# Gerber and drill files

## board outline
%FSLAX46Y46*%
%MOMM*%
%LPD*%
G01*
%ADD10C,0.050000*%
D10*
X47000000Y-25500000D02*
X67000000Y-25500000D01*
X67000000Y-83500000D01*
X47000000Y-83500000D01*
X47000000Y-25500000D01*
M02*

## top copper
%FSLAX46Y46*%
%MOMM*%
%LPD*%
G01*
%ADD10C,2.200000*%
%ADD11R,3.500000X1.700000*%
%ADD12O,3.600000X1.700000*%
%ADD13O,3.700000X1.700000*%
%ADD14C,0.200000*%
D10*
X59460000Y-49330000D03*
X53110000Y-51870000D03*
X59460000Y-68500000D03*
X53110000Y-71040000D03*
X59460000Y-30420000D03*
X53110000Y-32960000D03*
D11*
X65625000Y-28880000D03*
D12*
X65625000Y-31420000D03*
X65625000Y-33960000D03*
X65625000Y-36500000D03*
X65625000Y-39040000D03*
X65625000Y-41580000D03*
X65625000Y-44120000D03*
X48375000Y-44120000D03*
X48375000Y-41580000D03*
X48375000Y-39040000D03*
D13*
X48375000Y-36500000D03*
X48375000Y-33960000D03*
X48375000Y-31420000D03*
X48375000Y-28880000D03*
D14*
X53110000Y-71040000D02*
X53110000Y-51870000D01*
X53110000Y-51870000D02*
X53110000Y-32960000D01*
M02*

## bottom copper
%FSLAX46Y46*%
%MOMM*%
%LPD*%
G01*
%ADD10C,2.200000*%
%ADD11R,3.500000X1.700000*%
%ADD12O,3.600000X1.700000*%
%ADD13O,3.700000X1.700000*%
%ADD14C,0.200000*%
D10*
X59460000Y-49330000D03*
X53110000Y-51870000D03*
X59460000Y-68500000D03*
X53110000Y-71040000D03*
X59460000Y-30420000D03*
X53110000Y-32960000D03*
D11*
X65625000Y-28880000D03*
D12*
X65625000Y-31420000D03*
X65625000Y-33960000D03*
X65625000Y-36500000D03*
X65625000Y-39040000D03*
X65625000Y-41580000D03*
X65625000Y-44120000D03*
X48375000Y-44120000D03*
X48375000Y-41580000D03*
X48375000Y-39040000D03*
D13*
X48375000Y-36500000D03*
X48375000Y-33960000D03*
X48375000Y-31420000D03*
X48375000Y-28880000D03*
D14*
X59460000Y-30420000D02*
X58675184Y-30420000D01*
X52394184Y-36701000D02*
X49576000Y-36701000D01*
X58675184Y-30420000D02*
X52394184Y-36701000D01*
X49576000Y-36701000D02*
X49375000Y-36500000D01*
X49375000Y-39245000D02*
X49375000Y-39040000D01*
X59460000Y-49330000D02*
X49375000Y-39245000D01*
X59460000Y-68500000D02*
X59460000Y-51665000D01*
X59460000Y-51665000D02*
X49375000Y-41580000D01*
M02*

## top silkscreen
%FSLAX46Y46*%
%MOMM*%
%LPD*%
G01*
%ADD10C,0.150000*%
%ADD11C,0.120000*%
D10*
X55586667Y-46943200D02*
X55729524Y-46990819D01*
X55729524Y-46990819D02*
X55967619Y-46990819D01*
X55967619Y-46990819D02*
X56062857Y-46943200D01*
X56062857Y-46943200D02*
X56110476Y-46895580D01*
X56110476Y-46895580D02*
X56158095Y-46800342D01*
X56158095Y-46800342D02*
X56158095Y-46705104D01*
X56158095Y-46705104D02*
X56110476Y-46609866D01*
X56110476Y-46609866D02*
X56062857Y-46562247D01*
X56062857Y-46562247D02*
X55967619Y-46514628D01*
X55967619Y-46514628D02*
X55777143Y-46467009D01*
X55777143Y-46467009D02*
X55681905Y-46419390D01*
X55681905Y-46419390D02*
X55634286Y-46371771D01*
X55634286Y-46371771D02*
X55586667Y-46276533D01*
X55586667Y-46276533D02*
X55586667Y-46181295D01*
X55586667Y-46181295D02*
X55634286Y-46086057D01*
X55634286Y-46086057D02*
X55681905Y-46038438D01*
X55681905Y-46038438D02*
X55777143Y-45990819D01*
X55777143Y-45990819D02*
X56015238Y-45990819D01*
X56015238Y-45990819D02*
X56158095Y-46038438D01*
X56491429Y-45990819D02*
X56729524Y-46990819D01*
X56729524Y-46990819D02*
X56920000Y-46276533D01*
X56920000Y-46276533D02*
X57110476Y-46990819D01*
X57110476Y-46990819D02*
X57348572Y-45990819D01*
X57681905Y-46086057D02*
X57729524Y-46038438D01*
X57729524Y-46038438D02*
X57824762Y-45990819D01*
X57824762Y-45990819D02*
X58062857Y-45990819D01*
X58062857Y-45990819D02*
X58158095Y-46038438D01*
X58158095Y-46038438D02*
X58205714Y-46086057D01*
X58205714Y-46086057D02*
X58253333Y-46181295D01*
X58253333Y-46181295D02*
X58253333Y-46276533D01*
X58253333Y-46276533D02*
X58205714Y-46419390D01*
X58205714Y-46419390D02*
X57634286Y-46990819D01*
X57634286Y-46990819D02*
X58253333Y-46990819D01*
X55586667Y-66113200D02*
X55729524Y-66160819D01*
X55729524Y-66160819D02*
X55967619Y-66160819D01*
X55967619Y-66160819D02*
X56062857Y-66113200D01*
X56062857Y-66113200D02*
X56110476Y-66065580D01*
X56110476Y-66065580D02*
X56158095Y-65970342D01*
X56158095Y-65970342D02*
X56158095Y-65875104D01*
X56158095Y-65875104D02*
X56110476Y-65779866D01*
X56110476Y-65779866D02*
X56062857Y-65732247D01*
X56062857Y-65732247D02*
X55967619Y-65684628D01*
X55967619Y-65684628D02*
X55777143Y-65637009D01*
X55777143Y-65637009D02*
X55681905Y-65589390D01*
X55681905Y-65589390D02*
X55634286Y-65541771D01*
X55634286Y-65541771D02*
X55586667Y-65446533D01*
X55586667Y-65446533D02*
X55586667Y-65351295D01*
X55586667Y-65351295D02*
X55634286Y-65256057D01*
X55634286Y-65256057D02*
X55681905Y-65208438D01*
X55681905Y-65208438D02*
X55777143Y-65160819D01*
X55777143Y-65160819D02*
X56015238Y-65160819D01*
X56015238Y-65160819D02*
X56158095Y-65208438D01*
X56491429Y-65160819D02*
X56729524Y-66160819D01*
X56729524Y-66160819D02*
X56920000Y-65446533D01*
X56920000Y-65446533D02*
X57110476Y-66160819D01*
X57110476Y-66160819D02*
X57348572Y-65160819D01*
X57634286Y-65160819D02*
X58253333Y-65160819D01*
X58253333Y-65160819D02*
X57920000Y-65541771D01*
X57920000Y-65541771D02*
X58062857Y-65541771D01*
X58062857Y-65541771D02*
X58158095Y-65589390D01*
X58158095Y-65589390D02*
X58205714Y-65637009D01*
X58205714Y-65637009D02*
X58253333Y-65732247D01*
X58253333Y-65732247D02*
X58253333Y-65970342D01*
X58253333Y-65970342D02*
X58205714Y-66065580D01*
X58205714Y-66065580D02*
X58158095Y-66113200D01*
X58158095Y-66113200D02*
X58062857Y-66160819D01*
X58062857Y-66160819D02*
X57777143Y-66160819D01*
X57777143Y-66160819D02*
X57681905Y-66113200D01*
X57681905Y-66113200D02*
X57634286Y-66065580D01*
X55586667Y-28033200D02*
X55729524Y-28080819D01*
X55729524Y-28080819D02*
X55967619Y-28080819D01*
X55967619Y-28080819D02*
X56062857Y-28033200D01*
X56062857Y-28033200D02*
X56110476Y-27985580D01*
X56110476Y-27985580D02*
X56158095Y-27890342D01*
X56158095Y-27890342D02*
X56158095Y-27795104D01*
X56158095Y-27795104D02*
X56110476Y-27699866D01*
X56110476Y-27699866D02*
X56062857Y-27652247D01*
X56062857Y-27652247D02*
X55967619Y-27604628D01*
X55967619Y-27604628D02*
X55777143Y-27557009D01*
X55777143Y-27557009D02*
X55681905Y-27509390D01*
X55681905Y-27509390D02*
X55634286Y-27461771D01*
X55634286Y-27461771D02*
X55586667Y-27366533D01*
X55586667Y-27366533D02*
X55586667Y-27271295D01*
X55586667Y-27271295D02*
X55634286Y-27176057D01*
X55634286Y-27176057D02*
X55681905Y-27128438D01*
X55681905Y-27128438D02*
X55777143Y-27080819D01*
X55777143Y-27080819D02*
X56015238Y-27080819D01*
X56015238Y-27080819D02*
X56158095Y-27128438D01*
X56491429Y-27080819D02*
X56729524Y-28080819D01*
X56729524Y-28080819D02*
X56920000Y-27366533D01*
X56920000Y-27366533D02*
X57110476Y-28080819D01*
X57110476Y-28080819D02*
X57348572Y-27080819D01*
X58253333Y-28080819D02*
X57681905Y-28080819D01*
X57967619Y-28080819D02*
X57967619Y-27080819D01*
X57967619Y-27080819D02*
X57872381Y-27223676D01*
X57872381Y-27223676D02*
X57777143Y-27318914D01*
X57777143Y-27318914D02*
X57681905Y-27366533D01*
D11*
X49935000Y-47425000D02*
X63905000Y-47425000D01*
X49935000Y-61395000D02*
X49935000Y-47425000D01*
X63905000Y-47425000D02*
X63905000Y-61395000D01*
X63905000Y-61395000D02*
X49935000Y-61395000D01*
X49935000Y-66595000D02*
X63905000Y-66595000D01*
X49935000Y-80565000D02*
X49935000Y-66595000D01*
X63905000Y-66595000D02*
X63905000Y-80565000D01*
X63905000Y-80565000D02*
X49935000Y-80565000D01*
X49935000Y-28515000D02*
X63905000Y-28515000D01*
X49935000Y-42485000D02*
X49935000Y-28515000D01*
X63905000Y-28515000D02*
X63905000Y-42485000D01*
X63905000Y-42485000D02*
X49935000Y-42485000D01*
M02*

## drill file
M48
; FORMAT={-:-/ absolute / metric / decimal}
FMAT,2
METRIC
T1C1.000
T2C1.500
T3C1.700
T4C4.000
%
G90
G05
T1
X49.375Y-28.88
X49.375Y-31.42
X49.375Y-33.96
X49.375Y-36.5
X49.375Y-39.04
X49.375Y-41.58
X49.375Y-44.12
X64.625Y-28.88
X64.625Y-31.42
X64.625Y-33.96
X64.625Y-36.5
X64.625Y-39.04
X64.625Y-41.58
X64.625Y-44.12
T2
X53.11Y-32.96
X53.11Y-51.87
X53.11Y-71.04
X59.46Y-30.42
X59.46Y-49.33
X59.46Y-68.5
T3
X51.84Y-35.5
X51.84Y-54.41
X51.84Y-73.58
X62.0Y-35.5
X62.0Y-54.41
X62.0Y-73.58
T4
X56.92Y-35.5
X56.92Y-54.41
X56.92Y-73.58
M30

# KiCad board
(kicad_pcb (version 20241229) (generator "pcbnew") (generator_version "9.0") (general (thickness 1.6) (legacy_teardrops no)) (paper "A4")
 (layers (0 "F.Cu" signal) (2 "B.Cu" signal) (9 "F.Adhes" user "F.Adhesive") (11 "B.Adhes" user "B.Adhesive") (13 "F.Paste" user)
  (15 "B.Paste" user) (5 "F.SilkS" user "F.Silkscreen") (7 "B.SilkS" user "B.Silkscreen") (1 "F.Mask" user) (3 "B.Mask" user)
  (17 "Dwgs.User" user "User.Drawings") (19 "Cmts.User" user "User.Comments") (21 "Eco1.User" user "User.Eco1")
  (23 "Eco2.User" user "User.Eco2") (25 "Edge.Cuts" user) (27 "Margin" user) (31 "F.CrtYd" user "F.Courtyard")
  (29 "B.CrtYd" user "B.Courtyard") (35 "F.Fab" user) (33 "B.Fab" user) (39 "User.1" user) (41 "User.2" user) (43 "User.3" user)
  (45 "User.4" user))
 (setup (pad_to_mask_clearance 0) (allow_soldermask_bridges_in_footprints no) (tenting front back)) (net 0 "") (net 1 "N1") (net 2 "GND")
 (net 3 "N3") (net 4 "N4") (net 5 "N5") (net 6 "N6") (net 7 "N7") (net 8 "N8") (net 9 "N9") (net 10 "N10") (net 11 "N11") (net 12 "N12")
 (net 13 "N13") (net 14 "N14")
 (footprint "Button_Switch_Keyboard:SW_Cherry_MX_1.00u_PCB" (layer "F.Cu") (at 59.46 49.33)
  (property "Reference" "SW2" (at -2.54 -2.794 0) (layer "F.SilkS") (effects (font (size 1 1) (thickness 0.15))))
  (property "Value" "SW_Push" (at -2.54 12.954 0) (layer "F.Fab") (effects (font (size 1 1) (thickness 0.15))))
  (fp_line (start -9.525 -1.905) (end 4.445 -1.905) (stroke (width 0.12) (type solid)) (layer "F.SilkS"))
  (fp_line (start -9.525 12.065) (end -9.525 -1.905) (stroke (width 0.12) (type solid)) (layer "F.SilkS"))
  (fp_line (start 4.445 -1.905) (end 4.445 12.065) (stroke (width 0.12) (type solid)) (layer "F.SilkS"))
  (fp_line (start 4.445 12.065) (end -9.525 12.065) (stroke (width 0.12) (type solid)) (layer "F.SilkS"))
  (pad "" np_thru_hole circle (at -7.62 5.08) (size 1.7 1.7) (drill 1.7) (layers "*.Cu" "*.Mask"))
  (pad "" np_thru_hole circle (at -2.54 5.08) (size 4 4) (drill 4) (layers "*.Cu" "*.Mask"))
  (pad "" np_thru_hole circle (at 2.54 5.08) (size 1.7 1.7) (drill 1.7) (layers "*.Cu" "*.Mask"))
  (pad "1" thru_hole circle (at 0 0) (size 2.2 2.2) (drill 1.5) (layers "*.Cu" "*.Mask") (remove_unused_layers no) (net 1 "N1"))
  (pad "2" thru_hole circle (at -6.35 2.54) (size 2.2 2.2) (drill 1.5) (layers "*.Cu" "*.Mask") (remove_unused_layers no) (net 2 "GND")))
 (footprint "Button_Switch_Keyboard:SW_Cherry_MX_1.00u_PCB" (layer "F.Cu") (at 59.46 68.5)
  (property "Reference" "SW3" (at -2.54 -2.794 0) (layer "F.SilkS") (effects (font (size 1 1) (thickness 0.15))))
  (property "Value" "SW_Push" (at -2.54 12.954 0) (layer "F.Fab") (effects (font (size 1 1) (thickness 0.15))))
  (fp_line (start -9.525 -1.905) (end 4.445 -1.905) (stroke (width 0.12) (type solid)) (layer "F.SilkS"))
  (fp_line (start -9.525 12.065) (end -9.525 -1.905) (stroke (width 0.12) (type solid)) (layer "F.SilkS"))
  (fp_line (start 4.445 -1.905) (end 4.445 12.065) (stroke (width 0.12) (type solid)) (layer "F.SilkS"))
  (fp_line (start 4.445 12.065) (end -9.525 12.065) (stroke (width 0.12) (type solid)) (layer "F.SilkS"))
  (pad "" np_thru_hole circle (at -7.62 5.08) (size 1.7 1.7) (drill 1.7) (layers "*.Cu" "*.Mask"))
  (pad "" np_thru_hole circle (at -2.54 5.08) (size 4 4) (drill 4) (layers "*.Cu" "*.Mask"))
  (pad "" np_thru_hole circle (at 2.54 5.08) (size 1.7 1.7) (drill 1.7) (layers "*.Cu" "*.Mask"))
  (pad "1" thru_hole circle (at 0 0) (size 2.2 2.2) (drill 1.5) (layers "*.Cu" "*.Mask") (remove_unused_layers no) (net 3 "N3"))
  (pad "2" thru_hole circle (at -6.35 2.54) (size 2.2 2.2) (drill 1.5) (layers "*.Cu" "*.Mask") (remove_unused_layers no) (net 2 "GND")))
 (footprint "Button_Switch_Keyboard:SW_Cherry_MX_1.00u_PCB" (layer "F.Cu") (at 59.46 30.42)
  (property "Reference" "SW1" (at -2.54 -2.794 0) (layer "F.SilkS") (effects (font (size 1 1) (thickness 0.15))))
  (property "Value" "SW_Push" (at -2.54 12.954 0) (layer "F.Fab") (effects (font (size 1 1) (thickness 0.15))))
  (fp_line (start -9.525 -1.905) (end 4.445 -1.905) (stroke (width 0.12) (type solid)) (layer "F.SilkS"))
  (fp_line (start -9.525 12.065) (end -9.525 -1.905) (stroke (width 0.12) (type solid)) (layer "F.SilkS"))
  (fp_line (start 4.445 -1.905) (end 4.445 12.065) (stroke (width 0.12) (type solid)) (layer "F.SilkS"))
  (fp_line (start 4.445 12.065) (end -9.525 12.065) (stroke (width 0.12) (type solid)) (layer "F.SilkS"))
  (pad "" np_thru_hole circle (at -7.62 5.08) (size 1.7 1.7) (drill 1.7) (layers "*.Cu" "*.Mask"))
  (pad "" np_thru_hole circle (at -2.54 5.08) (size 4 4) (drill 4) (layers "*.Cu" "*.Mask"))
  (pad "" np_thru_hole circle (at 2.54 5.08) (size 1.7 1.7) (drill 1.7) (layers "*.Cu" "*.Mask"))
  (pad "1" thru_hole circle (at 0 0) (size 2.2 2.2) (drill 1.5) (layers "*.Cu" "*.Mask") (remove_unused_layers no) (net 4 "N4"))
  (pad "2" thru_hole circle (at -6.35 2.54) (size 2.2 2.2) (drill 1.5) (layers "*.Cu" "*.Mask") (remove_unused_layers no) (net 2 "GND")))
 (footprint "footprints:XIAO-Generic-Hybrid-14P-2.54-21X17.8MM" (layer "B.Cu") (at 57 36.5 180)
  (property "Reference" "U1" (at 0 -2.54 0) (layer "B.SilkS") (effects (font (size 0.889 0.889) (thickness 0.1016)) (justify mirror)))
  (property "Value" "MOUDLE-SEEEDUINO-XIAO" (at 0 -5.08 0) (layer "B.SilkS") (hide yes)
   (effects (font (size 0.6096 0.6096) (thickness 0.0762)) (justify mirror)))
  (pad "1" thru_hole rect (at -7.625 7.62 180) (size 3.5 1.7) (drill 1 (offset -1 0)) (layers "*.Cu" "*.Mask") (remove_unused_layers no)
   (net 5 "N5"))
  (pad "2" thru_hole oval (at -7.625 5.08 180) (size 3.6 1.7) (drill 1 (offset -1 0)) (layers "*.Cu" "*.Mask") (remove_unused_layers no)
   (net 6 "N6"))
  (pad "3" thru_hole oval (at -7.625 2.54 180) (size 3.6 1.7) (drill 1 (offset -1 0)) (layers "*.Cu" "*.Mask") (remove_unused_layers no)
   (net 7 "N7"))
  (pad "4" thru_hole oval (at -7.625 0 180) (size 3.6 1.7) (drill 1 (offset -1 0)) (layers "*.Cu" "*.Mask") (remove_unused_layers no)
   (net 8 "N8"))
  (pad "5" thru_hole oval (at -7.625 -2.54 180) (size 3.6 1.7) (drill 1 (offset -1 0)) (layers "*.Cu" "*.Mask") (remove_unused_layers no)
   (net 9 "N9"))
  (pad "6" thru_hole oval (at -7.625 -5.08) (size 3.6 1.7) (drill 1 (offset 1 0)) (layers "*.Cu" "*.Mask") (remove_unused_layers no)
   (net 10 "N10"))
  (pad "7" thru_hole oval (at -7.625 -7.62 180) (size 3.6 1.7) (drill 1 (offset -1 0)) (layers "*.Cu" "*.Mask") (remove_unused_layers no)
   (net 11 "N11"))
  (pad "8" thru_hole oval (at 7.625 -7.62 180) (size 3.6 1.7) (drill 1 (offset 1 0)) (layers "*.Cu" "*.Mask") (remove_unused_layers no)
   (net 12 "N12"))
  (pad "9" thru_hole oval (at 7.625 -5.08 180) (size 3.6 1.7) (drill 1 (offset 1 0)) (layers "*.Cu" "*.Mask") (remove_unused_layers no)
   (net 3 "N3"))
  (pad "10" thru_hole oval (at 7.625 -2.54 180) (size 3.6 1.7) (drill 1 (offset 1 0)) (layers "*.Cu" "*.Mask") (remove_unused_layers no)
   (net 1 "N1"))
  (pad "11" thru_hole oval (at 7.625 0 180) (size 3.7 1.7) (drill 1 (offset 1 0)) (layers "*.Cu" "*.Mask") (remove_unused_layers no)
   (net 4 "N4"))
  (pad "12" thru_hole oval (at 7.625 2.54 180) (size 3.7 1.7) (drill 1 (offset 1 0)) (layers "*.Cu" "*.Mask") (remove_unused_layers no)
   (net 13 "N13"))
  (pad "13" thru_hole oval (at 7.625 5.08 180) (size 3.7 1.7) (drill 1 (offset 1 0)) (layers "*.Cu" "*.Mask") (remove_unused_layers no)
   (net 2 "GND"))
  (pad "14" thru_hole oval (at 7.625 7.62 180) (size 3.7 1.7) (drill 1 (offset 1 0)) (layers "*.Cu" "*.Mask") (remove_unused_layers no)
   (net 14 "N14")))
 (gr_rect (start 47 25.5) (end 67 83.5) (stroke (width 0.05) (type default)) (fill no) (layer "Edge.Cuts"))
 (segment (start 53.11 71.04) (end 53.11 51.87) (width 0.2) (layer "F.Cu") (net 2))
 (segment (start 53.11 51.87) (end 53.11 32.96) (width 0.2) (layer "F.Cu") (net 2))
 (segment (start 59.46 30.42) (end 58.675184 30.42) (width 0.2) (layer "B.Cu") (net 4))
 (segment (start 52.394184 36.701) (end 49.576 36.701) (width 0.2) (layer "B.Cu") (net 4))
 (segment (start 58.675184 30.42) (end 52.394184 36.701) (width 0.2) (layer "B.Cu") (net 4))
 (segment (start 49.576 36.701) (end 49.375 36.5) (width 0.2) (layer "B.Cu") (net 4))
 (segment (start 49.375 39.245) (end 49.375 39.04) (width 0.2) (layer "B.Cu") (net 1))
 (segment (start 59.46 49.33) (end 49.375 39.245) (width 0.2) (layer "B.Cu") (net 1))
 (segment (start 59.46 68.5) (end 59.46 51.665) (width 0.2) (layer "B.Cu") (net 3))
 (segment (start 59.46 51.665) (end 49.375 41.58) (width 0.2) (layer "B.Cu") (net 3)))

